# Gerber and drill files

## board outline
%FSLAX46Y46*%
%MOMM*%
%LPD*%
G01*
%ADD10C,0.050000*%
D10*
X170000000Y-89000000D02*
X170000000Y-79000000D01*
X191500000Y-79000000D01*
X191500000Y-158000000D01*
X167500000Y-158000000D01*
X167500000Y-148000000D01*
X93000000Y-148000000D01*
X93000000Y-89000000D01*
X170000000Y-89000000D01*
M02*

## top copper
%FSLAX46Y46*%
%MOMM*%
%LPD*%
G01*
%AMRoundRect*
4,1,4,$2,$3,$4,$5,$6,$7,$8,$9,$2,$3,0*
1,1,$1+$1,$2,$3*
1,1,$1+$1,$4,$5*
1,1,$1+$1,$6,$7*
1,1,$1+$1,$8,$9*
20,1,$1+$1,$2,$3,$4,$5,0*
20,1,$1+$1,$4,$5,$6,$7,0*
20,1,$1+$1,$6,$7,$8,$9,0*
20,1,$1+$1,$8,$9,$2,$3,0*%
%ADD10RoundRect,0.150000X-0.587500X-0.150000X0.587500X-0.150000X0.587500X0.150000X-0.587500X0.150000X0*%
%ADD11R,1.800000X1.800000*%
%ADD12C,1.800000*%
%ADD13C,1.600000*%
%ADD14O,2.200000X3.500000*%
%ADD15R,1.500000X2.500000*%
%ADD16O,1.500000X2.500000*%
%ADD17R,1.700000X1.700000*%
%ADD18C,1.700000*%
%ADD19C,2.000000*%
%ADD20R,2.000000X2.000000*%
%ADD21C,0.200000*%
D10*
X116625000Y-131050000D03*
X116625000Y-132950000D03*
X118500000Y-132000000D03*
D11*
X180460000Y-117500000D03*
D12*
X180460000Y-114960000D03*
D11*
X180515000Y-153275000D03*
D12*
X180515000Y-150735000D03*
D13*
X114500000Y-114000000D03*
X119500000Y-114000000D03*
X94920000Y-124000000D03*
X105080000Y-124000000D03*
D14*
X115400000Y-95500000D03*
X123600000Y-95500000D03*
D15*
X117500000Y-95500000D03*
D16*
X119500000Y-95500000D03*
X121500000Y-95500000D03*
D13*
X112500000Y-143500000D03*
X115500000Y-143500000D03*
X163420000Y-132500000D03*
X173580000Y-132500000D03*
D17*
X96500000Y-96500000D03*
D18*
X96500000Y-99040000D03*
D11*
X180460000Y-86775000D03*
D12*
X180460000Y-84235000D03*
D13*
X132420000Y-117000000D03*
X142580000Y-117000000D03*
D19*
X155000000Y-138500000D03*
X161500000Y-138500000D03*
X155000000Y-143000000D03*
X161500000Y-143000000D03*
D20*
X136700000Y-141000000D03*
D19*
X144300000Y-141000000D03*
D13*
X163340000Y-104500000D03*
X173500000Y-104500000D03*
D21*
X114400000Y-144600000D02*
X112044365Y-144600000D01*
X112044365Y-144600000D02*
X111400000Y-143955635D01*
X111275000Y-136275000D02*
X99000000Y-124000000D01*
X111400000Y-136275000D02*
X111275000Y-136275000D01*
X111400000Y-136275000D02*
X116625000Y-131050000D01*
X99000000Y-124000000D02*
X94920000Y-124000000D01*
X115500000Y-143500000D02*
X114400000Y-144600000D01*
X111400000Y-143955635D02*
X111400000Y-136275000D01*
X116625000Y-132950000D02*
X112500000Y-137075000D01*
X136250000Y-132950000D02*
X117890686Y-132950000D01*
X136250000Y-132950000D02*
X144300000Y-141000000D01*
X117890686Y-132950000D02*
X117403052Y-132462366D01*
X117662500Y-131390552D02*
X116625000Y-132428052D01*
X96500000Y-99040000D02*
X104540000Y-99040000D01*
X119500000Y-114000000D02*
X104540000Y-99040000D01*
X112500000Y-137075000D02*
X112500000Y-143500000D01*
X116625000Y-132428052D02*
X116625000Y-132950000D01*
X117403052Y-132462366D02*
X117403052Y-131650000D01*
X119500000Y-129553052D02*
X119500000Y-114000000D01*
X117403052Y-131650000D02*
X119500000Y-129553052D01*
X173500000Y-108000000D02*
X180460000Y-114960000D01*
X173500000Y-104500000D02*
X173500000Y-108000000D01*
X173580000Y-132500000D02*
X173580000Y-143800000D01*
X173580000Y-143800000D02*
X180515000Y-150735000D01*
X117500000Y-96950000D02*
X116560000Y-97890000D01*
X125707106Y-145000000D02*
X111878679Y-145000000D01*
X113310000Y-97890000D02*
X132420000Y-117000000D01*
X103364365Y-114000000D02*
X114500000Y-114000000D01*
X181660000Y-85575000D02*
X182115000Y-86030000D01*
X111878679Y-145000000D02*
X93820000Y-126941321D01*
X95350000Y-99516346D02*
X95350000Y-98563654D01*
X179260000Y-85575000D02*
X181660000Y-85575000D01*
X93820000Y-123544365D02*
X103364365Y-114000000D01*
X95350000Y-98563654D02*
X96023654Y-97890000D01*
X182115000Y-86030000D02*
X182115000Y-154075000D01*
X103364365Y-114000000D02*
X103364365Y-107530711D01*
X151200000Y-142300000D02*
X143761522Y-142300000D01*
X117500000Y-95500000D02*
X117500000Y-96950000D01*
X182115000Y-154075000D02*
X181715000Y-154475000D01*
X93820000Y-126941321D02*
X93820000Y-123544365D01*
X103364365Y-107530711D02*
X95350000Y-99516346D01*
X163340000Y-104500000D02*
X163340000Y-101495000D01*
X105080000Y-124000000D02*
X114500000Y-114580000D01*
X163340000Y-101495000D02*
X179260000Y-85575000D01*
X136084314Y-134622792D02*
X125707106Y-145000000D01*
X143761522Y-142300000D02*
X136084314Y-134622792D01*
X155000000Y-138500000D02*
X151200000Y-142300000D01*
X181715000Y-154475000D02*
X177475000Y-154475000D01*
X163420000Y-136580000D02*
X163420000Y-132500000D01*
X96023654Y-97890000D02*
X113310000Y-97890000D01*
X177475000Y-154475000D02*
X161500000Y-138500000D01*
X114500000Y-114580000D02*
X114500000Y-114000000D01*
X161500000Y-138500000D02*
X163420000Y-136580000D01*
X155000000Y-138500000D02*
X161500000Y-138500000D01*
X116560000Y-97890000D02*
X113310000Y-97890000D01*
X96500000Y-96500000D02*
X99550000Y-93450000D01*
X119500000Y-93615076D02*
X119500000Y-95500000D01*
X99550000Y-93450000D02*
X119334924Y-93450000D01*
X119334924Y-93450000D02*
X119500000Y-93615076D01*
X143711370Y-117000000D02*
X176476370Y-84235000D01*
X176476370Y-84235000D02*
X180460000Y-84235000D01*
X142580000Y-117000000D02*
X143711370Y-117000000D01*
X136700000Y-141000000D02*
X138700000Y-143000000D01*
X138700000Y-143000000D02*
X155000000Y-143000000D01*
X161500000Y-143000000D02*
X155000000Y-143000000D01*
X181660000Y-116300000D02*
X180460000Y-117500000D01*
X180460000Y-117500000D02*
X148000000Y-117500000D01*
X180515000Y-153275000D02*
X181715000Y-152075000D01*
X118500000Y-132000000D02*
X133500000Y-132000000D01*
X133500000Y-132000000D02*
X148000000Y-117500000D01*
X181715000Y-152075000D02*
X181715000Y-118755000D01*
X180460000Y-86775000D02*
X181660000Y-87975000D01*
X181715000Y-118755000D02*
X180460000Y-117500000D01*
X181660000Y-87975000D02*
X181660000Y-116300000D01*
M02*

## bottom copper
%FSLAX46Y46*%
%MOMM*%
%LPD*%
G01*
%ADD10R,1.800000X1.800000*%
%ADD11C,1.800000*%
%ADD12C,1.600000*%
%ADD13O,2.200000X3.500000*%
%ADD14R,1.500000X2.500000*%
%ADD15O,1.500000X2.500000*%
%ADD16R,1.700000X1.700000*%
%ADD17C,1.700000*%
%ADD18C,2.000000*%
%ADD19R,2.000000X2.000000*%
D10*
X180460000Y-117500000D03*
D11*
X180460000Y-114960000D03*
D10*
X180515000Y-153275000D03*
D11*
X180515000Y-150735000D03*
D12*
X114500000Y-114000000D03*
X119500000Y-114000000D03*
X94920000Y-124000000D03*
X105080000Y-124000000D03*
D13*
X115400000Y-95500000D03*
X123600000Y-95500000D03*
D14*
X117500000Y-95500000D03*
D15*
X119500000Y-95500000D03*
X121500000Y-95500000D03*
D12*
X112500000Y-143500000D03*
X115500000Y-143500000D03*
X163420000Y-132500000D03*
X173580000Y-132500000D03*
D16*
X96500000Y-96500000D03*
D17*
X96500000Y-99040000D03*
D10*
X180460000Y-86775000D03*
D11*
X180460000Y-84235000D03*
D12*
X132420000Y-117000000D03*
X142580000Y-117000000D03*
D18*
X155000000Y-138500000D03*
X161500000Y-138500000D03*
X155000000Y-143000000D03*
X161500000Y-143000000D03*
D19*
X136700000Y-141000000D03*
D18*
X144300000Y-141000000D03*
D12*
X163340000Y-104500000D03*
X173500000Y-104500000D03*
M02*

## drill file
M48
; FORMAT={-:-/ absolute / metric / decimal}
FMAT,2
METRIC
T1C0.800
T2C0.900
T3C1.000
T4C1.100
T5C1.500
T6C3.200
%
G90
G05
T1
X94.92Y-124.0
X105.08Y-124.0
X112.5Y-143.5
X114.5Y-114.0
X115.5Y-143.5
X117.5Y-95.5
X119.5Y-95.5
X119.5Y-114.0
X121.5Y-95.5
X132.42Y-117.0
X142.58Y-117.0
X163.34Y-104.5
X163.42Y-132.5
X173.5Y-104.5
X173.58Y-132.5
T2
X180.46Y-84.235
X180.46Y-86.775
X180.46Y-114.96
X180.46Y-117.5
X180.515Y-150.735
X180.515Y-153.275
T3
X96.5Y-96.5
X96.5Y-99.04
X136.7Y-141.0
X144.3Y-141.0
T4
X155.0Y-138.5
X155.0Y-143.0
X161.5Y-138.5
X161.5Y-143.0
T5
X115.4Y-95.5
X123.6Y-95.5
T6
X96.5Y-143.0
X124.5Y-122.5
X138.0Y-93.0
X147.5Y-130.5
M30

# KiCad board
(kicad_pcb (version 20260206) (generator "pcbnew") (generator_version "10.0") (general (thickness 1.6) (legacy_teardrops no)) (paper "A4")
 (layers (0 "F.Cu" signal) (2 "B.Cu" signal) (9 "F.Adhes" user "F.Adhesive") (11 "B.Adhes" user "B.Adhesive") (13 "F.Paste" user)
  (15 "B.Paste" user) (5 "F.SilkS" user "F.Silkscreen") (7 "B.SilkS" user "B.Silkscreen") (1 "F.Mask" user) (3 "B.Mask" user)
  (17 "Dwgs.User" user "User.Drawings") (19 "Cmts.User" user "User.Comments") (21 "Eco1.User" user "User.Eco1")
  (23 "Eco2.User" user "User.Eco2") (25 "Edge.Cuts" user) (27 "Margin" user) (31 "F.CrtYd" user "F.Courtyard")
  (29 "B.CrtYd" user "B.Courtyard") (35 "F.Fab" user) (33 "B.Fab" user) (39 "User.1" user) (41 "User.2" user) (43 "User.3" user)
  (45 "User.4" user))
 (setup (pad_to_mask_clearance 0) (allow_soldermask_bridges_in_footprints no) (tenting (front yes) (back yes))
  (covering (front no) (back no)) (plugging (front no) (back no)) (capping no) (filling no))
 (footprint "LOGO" (layer "F.Cu") (at 137.5 102.5)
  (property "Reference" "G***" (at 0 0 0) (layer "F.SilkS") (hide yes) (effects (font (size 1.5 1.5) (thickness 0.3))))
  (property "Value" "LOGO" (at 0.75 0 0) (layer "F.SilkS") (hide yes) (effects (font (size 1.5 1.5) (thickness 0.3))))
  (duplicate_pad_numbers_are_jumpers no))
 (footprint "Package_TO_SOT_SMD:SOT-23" (layer "F.Cu") (at 117.5625 132)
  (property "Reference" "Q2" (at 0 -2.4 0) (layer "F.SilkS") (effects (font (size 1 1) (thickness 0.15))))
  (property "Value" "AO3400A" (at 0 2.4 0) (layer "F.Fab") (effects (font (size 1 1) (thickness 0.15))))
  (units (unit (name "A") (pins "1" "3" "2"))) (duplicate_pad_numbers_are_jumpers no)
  (pad "1" smd roundrect (at -0.9375 -0.95) (size 1.475 0.6) (layers "F.Cu" "F.Mask" "F.Paste") (roundrect_rratio 0.25) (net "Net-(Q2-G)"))
  (pad "2" smd roundrect (at -0.9375 0.95) (size 1.475 0.6) (layers "F.Cu" "F.Mask" "F.Paste") (roundrect_rratio 0.25) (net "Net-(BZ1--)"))
  (pad "3" smd roundrect (at 0.9375 0) (size 1.475 0.6) (layers "F.Cu" "F.Mask" "F.Paste") (roundrect_rratio 0.25) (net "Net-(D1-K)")))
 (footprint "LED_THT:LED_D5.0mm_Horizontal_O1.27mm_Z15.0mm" (layer "F.Cu") (at 180.46 117.5 90)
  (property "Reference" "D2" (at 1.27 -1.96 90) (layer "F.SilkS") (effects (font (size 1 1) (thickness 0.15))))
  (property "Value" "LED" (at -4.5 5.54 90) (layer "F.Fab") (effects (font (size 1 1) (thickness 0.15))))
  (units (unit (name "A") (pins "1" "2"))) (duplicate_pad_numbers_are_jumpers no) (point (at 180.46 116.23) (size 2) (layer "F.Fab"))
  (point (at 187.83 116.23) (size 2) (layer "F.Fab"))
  (pad "1" thru_hole rect (at 0 0 90) (size 1.8 1.8) (drill 0.9) (layers "*.Cu" "*.Mask") (remove_unused_layers no) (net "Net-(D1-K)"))
  (pad "2" thru_hole circle (at 2.54 0 90) (size 1.8 1.8) (drill 0.9) (layers "*.Cu" "*.Mask") (remove_unused_layers no) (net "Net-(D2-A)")))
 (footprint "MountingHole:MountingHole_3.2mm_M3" (layer "F.Cu") (at 138 93)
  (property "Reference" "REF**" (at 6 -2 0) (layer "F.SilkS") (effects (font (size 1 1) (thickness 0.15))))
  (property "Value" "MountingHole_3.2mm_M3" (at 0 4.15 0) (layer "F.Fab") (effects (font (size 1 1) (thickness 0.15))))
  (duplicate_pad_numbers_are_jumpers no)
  (pad "" np_thru_hole circle (at 0 0) (size 3.2 3.2) (drill 3.2) (layers "*.Cu" "*.Mask")))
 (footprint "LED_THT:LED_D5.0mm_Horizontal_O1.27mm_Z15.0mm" (layer "F.Cu") (at 180.515 153.275 90)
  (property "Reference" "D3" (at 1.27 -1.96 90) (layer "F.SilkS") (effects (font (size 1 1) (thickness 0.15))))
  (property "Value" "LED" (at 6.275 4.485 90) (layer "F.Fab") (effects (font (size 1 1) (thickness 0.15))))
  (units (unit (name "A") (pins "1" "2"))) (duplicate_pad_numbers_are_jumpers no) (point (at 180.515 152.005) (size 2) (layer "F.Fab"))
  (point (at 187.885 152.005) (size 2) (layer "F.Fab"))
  (pad "1" thru_hole rect (at 0 0 90) (size 1.8 1.8) (drill 0.9) (layers "*.Cu" "*.Mask") (remove_unused_layers no) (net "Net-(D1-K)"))
  (pad "2" thru_hole circle (at 2.54 0 90) (size 1.8 1.8) (drill 0.9) (layers "*.Cu" "*.Mask") (remove_unused_layers no) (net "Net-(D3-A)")))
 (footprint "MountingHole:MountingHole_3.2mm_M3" (layer "F.Cu") (at 147.5 130.5)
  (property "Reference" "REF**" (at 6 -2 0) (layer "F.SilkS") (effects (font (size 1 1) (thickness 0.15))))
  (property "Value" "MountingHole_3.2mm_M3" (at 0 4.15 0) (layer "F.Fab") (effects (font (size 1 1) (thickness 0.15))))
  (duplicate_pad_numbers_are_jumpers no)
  (pad "" np_thru_hole circle (at 0 0) (size 3.2 3.2) (drill 3.2) (layers "*.Cu" "*.Mask")))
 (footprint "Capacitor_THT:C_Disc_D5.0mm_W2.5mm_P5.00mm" (layer "F.Cu") (at 114.5 114)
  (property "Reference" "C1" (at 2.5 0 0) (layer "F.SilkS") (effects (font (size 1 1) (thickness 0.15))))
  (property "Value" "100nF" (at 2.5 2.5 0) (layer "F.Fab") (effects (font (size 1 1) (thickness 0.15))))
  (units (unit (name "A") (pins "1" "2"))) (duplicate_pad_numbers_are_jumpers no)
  (pad "1" thru_hole circle (at 0 0) (size 1.6 1.6) (drill 0.8) (layers "*.Cu" "*.Mask") (remove_unused_layers no) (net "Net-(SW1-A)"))
  (pad "2" thru_hole circle (at 5 0) (size 1.6 1.6) (drill 0.8) (layers "*.Cu" "*.Mask") (remove_unused_layers no) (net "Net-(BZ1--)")))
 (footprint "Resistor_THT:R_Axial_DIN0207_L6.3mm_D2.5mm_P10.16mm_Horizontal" (layer "F.Cu") (at 94.92 124)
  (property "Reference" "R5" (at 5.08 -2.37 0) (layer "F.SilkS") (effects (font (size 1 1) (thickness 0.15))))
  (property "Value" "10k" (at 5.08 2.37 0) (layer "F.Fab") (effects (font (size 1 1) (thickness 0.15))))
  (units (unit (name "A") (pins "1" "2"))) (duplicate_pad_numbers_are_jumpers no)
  (pad "1" thru_hole circle (at 0 0) (size 1.6 1.6) (drill 0.8) (layers "*.Cu" "*.Mask") (remove_unused_layers no) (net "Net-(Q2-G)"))
  (pad "2" thru_hole circle (at 10.16 0) (size 1.6 1.6) (drill 0.8) (layers "*.Cu" "*.Mask") (remove_unused_layers no) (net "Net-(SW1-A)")))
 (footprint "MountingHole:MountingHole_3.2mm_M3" (layer "F.Cu") (at 124.5 122.5)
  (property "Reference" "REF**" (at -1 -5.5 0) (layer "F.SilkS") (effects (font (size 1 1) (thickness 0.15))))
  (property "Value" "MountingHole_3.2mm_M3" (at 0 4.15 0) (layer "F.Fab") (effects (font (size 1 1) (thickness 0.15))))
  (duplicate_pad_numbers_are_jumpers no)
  (pad "" np_thru_hole circle (at 0 0) (size 3.2 3.2) (drill 3.2) (layers "*.Cu" "*.Mask")))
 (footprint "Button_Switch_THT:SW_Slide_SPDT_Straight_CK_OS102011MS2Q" (layer "F.Cu") (at 117.5 95.5)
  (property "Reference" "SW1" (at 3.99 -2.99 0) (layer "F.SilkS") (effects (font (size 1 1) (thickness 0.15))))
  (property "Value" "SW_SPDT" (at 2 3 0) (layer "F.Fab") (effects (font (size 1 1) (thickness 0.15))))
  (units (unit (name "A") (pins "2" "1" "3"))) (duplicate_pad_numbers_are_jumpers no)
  (pad "" thru_hole oval (at -2.1 0) (size 2.2 3.5) (drill 1.5) (layers "*.Cu" "*.Mask") (remove_unused_layers no))
  (pad "" thru_hole oval (at 6.1 0) (size 2.2 3.5) (drill 1.5) (layers "*.Cu" "*.Mask") (remove_unused_layers no))
  (pad "1" thru_hole rect (at 0 0) (size 1.5 2.5) (drill 0.8) (layers "*.Cu" "*.Mask") (remove_unused_layers no) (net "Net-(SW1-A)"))
  (pad "2" thru_hole oval (at 2 0) (size 1.5 2.5) (drill 0.8) (layers "*.Cu" "*.Mask") (remove_unused_layers no) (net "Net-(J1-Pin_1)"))
  (pad "3" thru_hole oval (at 4 0) (size 1.5 2.5) (drill 0.8) (layers "*.Cu" "*.Mask") (remove_unused_layers no)
   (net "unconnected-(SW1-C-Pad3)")))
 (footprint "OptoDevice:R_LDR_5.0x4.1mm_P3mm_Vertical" (layer "F.Cu") (at 112.5 143.5)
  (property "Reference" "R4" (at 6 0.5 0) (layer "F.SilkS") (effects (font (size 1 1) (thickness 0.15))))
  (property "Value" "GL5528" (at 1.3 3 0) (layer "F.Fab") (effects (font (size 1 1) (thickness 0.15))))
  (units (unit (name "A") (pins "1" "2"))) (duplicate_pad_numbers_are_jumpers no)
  (pad "1" thru_hole circle (at 0 0) (size 1.6 1.6) (drill 0.8) (layers "*.Cu" "*.Mask") (remove_unused_layers no) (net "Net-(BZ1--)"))
  (pad "2" thru_hole circle (at 3 0) (size 1.6 1.6) (drill 0.8) (layers "*.Cu" "*.Mask") (remove_unused_layers no) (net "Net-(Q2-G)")))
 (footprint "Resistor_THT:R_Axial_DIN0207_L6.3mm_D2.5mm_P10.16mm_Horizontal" (layer "F.Cu") (at 163.42 132.5)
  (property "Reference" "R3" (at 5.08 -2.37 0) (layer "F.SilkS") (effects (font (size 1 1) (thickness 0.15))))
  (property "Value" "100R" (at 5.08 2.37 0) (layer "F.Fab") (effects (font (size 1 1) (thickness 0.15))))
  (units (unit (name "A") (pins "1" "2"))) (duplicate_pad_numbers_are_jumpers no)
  (pad "1" thru_hole circle (at 0 0) (size 1.6 1.6) (drill 0.8) (layers "*.Cu" "*.Mask") (remove_unused_layers no) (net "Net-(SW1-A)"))
  (pad "2" thru_hole circle (at 10.16 0) (size 1.6 1.6) (drill 0.8) (layers "*.Cu" "*.Mask") (remove_unused_layers no) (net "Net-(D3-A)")))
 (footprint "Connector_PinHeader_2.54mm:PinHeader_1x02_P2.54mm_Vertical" (layer "F.Cu") (at 96.5 96.5)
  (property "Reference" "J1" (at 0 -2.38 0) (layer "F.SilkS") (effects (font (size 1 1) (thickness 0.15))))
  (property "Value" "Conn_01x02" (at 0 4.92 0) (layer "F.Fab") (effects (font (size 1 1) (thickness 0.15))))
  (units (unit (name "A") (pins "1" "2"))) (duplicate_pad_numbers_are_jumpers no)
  (pad "1" thru_hole rect (at 0 0) (size 1.7 1.7) (drill 1) (layers "*.Cu" "*.Mask") (remove_unused_layers no) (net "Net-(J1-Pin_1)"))
  (pad "2" thru_hole circle (at 0 2.54) (size 1.7 1.7) (drill 1) (layers "*.Cu" "*.Mask") (remove_unused_layers no) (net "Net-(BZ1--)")))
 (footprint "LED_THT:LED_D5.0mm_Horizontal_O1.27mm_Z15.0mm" (layer "F.Cu") (at 180.46 86.775 90)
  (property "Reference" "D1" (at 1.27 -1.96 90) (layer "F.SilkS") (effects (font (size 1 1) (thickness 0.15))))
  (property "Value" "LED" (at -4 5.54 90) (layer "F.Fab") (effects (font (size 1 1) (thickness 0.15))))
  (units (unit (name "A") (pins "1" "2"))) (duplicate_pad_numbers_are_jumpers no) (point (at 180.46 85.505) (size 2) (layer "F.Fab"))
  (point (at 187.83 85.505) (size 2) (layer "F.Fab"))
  (pad "1" thru_hole rect (at 0 0 90) (size 1.8 1.8) (drill 0.9) (layers "*.Cu" "*.Mask") (remove_unused_layers no) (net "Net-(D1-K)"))
  (pad "2" thru_hole circle (at 2.54 0 90) (size 1.8 1.8) (drill 0.9) (layers "*.Cu" "*.Mask") (remove_unused_layers no) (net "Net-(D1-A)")))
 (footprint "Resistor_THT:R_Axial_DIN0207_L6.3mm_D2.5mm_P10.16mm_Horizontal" (layer "F.Cu") (at 132.42 117)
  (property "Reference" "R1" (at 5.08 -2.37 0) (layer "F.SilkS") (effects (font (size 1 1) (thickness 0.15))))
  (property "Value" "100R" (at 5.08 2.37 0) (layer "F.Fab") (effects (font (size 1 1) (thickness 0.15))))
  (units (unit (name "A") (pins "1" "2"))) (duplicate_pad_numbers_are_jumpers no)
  (pad "1" thru_hole circle (at 0 0) (size 1.6 1.6) (drill 0.8) (layers "*.Cu" "*.Mask") (remove_unused_layers no) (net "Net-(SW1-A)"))
  (pad "2" thru_hole circle (at 10.16 0) (size 1.6 1.6) (drill 0.8) (layers "*.Cu" "*.Mask") (remove_unused_layers no) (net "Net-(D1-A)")))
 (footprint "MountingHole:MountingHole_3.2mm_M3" (layer "F.Cu") (at 96.5 143)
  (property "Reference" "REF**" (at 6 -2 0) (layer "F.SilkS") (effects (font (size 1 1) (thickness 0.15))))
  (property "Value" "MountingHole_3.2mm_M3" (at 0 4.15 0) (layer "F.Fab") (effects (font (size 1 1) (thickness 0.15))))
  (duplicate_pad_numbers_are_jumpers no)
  (pad "" np_thru_hole circle (at 0 0) (size 3.2 3.2) (drill 3.2) (layers "*.Cu" "*.Mask")))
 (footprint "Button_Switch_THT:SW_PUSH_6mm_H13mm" (layer "F.Cu") (at 155 138.5)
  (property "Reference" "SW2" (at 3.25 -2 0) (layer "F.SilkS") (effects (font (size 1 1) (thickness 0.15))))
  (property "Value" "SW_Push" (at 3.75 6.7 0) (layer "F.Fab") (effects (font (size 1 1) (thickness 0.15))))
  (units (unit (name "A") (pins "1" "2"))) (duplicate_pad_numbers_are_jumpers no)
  (pad "1" thru_hole circle (at 0 0 90) (size 2 2) (drill 1.1) (layers "*.Cu" "*.Mask") (remove_unused_layers no) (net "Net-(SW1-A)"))
  (pad "1" thru_hole circle (at 6.5 0 90) (size 2 2) (drill 1.1) (layers "*.Cu" "*.Mask") (remove_unused_layers no) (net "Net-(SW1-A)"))
  (pad "2" thru_hole circle (at 0 4.5 90) (size 2 2) (drill 1.1) (layers "*.Cu" "*.Mask") (remove_unused_layers no) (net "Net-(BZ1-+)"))
  (pad "2" thru_hole circle (at 6.5 4.5 90) (size 2 2) (drill 1.1) (layers "*.Cu" "*.Mask") (remove_unused_layers no) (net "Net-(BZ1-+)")))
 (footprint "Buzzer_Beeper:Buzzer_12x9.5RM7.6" (layer "F.Cu") (at 136.7 141)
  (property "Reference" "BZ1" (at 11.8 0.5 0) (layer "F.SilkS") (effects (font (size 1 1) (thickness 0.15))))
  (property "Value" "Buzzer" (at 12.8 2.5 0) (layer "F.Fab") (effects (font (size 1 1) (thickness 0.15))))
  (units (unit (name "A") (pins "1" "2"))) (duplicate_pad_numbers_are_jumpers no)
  (pad "1" thru_hole rect (at 0 0) (size 2 2) (drill 1) (layers "*.Cu" "*.Mask") (remove_unused_layers no) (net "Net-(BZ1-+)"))
  (pad "2" thru_hole circle (at 7.6 0) (size 2 2) (drill 1) (layers "*.Cu" "*.Mask") (remove_unused_layers no) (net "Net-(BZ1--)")))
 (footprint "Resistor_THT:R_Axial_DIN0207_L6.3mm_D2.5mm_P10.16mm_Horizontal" (layer "F.Cu") (at 163.34 104.5)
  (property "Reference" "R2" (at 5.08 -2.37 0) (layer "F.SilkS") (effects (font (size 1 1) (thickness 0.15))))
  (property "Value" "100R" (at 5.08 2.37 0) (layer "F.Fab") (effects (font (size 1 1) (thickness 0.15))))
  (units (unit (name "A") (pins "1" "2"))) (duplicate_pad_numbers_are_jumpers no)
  (pad "1" thru_hole circle (at 0 0) (size 1.6 1.6) (drill 0.8) (layers "*.Cu" "*.Mask") (remove_unused_layers no) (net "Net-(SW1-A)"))
  (pad "2" thru_hole circle (at 10.16 0) (size 1.6 1.6) (drill 0.8) (layers "*.Cu" "*.Mask") (remove_unused_layers no) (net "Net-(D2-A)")))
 (gr_poly
  (pts (xy 170 89) (xy 170 79) (xy 191.5 79) (xy 191.5 158) (xy 167.5 158) (xy 167.5 148) (xy 93 148) (xy 93 89))
  (stroke (width 0.05) (type solid)) (fill no) (layer "Edge.Cuts"))
 (segment (start 114.4 144.6) (end 112.044365 144.6) (width 0.2) (layer "F.Cu") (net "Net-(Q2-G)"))
 (segment (start 112.044365 144.6) (end 111.4 143.955635) (width 0.2) (layer "F.Cu") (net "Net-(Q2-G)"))
 (segment (start 111.275 136.275) (end 99 124) (width 0.2) (layer "F.Cu") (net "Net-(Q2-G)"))
 (segment (start 111.4 136.275) (end 111.275 136.275) (width 0.2) (layer "F.Cu") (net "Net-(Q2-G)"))
 (segment (start 111.4 136.275) (end 116.625 131.05) (width 0.2) (layer "F.Cu") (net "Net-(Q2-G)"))
 (segment (start 99 124) (end 94.92 124) (width 0.2) (layer "F.Cu") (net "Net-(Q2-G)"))
 (segment (start 115.5 143.5) (end 114.4 144.6) (width 0.2) (layer "F.Cu") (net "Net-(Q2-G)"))
 (segment (start 111.4 143.955635) (end 111.4 136.275) (width 0.2) (layer "F.Cu") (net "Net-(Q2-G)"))
 (segment (start 116.625 132.95) (end 112.5 137.075) (width 0.2) (layer "F.Cu") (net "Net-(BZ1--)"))
 (segment (start 136.25 132.95) (end 117.890686 132.95) (width 0.2) (layer "F.Cu") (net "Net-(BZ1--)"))
 (segment (start 136.25 132.95) (end 144.3 141) (width 0.2) (layer "F.Cu") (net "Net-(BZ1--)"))
 (segment (start 117.890686 132.95) (end 117.403052 132.462366) (width 0.2) (layer "F.Cu") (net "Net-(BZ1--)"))
 (segment (start 117.6625 131.390552) (end 116.625 132.428052) (width 0.2) (layer "F.Cu") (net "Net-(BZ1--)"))
 (segment (start 96.5 99.04) (end 104.54 99.04) (width 0.2) (layer "F.Cu") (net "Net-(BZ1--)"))
 (segment (start 119.5 114) (end 104.54 99.04) (width 0.2) (layer "F.Cu") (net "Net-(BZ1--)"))
 (segment (start 112.5 137.075) (end 112.5 143.5) (width 0.2) (layer "F.Cu") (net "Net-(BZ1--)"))
 (segment (start 116.625 132.428052) (end 116.625 132.95) (width 0.2) (layer "F.Cu") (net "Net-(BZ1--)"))
 (segment (start 117.403052 132.462366) (end 117.403052 131.65) (width 0.2) (layer "F.Cu") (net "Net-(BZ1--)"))
 (segment (start 119.5 129.553052) (end 119.5 114) (width 0.2) (layer "F.Cu") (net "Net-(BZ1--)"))
 (segment (start 117.403052 131.65) (end 119.5 129.553052) (width 0.2) (layer "F.Cu") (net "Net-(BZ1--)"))
 (segment (start 173.5 108) (end 180.46 114.96) (width 0.2) (layer "F.Cu") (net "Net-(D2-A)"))
 (segment (start 173.5 104.5) (end 173.5 108) (width 0.2) (layer "F.Cu") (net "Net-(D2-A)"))
 (segment (start 173.58 132.5) (end 173.58 143.8) (width 0.2) (layer "F.Cu") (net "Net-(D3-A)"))
 (segment (start 173.58 143.8) (end 180.515 150.735) (width 0.2) (layer "F.Cu") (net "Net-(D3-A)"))
 (segment (start 117.5 96.95) (end 116.56 97.89) (width 0.2) (layer "F.Cu") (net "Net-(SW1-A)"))
 (segment (start 125.707106 145) (end 111.878679 145) (width 0.2) (layer "F.Cu") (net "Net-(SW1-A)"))
 (segment (start 113.31 97.89) (end 132.42 117) (width 0.2) (layer "F.Cu") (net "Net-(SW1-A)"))
 (segment (start 103.364365 114) (end 114.5 114) (width 0.2) (layer "F.Cu") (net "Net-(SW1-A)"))
 (segment (start 181.66 85.575) (end 182.115 86.03) (width 0.2) (layer "F.Cu") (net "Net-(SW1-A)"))
 (segment (start 111.878679 145) (end 93.82 126.941321) (width 0.2) (layer "F.Cu") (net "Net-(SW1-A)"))
 (segment (start 95.35 99.516346) (end 95.35 98.563654) (width 0.2) (layer "F.Cu") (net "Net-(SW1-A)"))
 (segment (start 179.26 85.575) (end 181.66 85.575) (width 0.2) (layer "F.Cu") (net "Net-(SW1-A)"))
 (segment (start 93.82 123.544365) (end 103.364365 114) (width 0.2) (layer "F.Cu") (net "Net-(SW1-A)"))
 (segment (start 95.35 98.563654) (end 96.023654 97.89) (width 0.2) (layer "F.Cu") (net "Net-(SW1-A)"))
 (segment (start 182.115 86.03) (end 182.115 154.075) (width 0.2) (layer "F.Cu") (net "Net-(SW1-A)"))
 (segment (start 103.364365 114) (end 103.364365 107.530711) (width 0.2) (layer "F.Cu") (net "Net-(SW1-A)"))
 (segment (start 151.2 142.3) (end 143.761522 142.3) (width 0.2) (layer "F.Cu") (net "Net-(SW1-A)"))
 (segment (start 117.5 95.5) (end 117.5 96.95) (width 0.2) (layer "F.Cu") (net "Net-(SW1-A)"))
 (segment (start 182.115 154.075) (end 181.715 154.475) (width 0.2) (layer "F.Cu") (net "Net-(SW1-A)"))
 (segment (start 93.82 126.941321) (end 93.82 123.544365) (width 0.2) (layer "F.Cu") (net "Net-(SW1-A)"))
 (segment (start 103.364365 107.530711) (end 95.35 99.516346) (width 0.2) (layer "F.Cu") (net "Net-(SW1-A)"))
 (segment (start 163.34 104.5) (end 163.34 101.495) (width 0.2) (layer "F.Cu") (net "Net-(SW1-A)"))
 (segment (start 105.08 124) (end 114.5 114.58) (width 0.2) (layer "F.Cu") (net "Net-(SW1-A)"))
 (segment (start 163.34 101.495) (end 179.26 85.575) (width 0.2) (layer "F.Cu") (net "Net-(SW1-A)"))
 (segment (start 136.084314 134.622792) (end 125.707106 145) (width 0.2) (layer "F.Cu") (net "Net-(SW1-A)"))
 (segment (start 143.761522 142.3) (end 136.084314 134.622792) (width 0.2) (layer "F.Cu") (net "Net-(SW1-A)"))
 (segment (start 155 138.5) (end 151.2 142.3) (width 0.2) (layer "F.Cu") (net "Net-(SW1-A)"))
 (segment (start 181.715 154.475) (end 177.475 154.475) (width 0.2) (layer "F.Cu") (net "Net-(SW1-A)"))
 (segment (start 163.42 136.58) (end 163.42 132.5) (width 0.2) (layer "F.Cu") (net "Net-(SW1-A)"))
 (segment (start 96.023654 97.89) (end 113.31 97.89) (width 0.2) (layer "F.Cu") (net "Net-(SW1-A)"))
 (segment (start 177.475 154.475) (end 161.5 138.5) (width 0.2) (layer "F.Cu") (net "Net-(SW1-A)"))
 (segment (start 114.5 114.58) (end 114.5 114) (width 0.2) (layer "F.Cu") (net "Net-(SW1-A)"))
 (segment (start 161.5 138.5) (end 163.42 136.58) (width 0.2) (layer "F.Cu") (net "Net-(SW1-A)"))
 (segment (start 155 138.5) (end 161.5 138.5) (width 0.2) (layer "F.Cu") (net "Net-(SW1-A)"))
 (segment (start 116.56 97.89) (end 113.31 97.89) (width 0.2) (layer "F.Cu") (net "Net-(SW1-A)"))
 (segment (start 96.5 96.5) (end 99.55 93.45) (width 0.2) (layer "F.Cu") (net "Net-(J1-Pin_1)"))
 (segment (start 119.5 93.615076) (end 119.5 95.5) (width 0.2) (layer "F.Cu") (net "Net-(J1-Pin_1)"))
 (segment (start 99.55 93.45) (end 119.334924 93.45) (width 0.2) (layer "F.Cu") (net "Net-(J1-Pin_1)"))
 (segment (start 119.334924 93.45) (end 119.5 93.615076) (width 0.2) (layer "F.Cu") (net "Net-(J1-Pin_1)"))
 (segment (start 143.71137 117) (end 176.47637 84.235) (width 0.2) (layer "F.Cu") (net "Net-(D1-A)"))
 (segment (start 176.47637 84.235) (end 180.46 84.235) (width 0.2) (layer "F.Cu") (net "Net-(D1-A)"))
 (segment (start 142.58 117) (end 143.71137 117) (width 0.2) (layer "F.Cu") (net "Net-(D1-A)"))
 (segment (start 136.7 141) (end 138.7 143) (width 0.2) (layer "F.Cu") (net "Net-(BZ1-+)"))
 (segment (start 138.7 143) (end 155 143) (width 0.2) (layer "F.Cu") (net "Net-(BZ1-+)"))
 (segment (start 161.5 143) (end 155 143) (width 0.2) (layer "F.Cu") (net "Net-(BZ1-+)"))
 (segment (start 181.66 116.3) (end 180.46 117.5) (width 0.2) (layer "F.Cu") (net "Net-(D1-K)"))
 (segment (start 180.46 117.5) (end 148 117.5) (width 0.2) (layer "F.Cu") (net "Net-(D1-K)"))
 (segment (start 180.515 153.275) (end 181.715 152.075) (width 0.2) (layer "F.Cu") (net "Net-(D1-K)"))
 (segment (start 118.5 132) (end 133.5 132) (width 0.2) (layer "F.Cu") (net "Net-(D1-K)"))
 (segment (start 133.5 132) (end 148 117.5) (width 0.2) (layer "F.Cu") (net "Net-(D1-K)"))
 (segment (start 181.715 152.075) (end 181.715 118.755) (width 0.2) (layer "F.Cu") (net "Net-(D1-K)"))
 (segment (start 180.46 86.775) (end 181.66 87.975) (width 0.2) (layer "F.Cu") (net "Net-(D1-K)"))
 (segment (start 181.715 118.755) (end 180.46 117.5) (width 0.2) (layer "F.Cu") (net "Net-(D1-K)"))
 (segment (start 181.66 87.975) (end 181.66 116.3) (width 0.2) (layer "F.Cu") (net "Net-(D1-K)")))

